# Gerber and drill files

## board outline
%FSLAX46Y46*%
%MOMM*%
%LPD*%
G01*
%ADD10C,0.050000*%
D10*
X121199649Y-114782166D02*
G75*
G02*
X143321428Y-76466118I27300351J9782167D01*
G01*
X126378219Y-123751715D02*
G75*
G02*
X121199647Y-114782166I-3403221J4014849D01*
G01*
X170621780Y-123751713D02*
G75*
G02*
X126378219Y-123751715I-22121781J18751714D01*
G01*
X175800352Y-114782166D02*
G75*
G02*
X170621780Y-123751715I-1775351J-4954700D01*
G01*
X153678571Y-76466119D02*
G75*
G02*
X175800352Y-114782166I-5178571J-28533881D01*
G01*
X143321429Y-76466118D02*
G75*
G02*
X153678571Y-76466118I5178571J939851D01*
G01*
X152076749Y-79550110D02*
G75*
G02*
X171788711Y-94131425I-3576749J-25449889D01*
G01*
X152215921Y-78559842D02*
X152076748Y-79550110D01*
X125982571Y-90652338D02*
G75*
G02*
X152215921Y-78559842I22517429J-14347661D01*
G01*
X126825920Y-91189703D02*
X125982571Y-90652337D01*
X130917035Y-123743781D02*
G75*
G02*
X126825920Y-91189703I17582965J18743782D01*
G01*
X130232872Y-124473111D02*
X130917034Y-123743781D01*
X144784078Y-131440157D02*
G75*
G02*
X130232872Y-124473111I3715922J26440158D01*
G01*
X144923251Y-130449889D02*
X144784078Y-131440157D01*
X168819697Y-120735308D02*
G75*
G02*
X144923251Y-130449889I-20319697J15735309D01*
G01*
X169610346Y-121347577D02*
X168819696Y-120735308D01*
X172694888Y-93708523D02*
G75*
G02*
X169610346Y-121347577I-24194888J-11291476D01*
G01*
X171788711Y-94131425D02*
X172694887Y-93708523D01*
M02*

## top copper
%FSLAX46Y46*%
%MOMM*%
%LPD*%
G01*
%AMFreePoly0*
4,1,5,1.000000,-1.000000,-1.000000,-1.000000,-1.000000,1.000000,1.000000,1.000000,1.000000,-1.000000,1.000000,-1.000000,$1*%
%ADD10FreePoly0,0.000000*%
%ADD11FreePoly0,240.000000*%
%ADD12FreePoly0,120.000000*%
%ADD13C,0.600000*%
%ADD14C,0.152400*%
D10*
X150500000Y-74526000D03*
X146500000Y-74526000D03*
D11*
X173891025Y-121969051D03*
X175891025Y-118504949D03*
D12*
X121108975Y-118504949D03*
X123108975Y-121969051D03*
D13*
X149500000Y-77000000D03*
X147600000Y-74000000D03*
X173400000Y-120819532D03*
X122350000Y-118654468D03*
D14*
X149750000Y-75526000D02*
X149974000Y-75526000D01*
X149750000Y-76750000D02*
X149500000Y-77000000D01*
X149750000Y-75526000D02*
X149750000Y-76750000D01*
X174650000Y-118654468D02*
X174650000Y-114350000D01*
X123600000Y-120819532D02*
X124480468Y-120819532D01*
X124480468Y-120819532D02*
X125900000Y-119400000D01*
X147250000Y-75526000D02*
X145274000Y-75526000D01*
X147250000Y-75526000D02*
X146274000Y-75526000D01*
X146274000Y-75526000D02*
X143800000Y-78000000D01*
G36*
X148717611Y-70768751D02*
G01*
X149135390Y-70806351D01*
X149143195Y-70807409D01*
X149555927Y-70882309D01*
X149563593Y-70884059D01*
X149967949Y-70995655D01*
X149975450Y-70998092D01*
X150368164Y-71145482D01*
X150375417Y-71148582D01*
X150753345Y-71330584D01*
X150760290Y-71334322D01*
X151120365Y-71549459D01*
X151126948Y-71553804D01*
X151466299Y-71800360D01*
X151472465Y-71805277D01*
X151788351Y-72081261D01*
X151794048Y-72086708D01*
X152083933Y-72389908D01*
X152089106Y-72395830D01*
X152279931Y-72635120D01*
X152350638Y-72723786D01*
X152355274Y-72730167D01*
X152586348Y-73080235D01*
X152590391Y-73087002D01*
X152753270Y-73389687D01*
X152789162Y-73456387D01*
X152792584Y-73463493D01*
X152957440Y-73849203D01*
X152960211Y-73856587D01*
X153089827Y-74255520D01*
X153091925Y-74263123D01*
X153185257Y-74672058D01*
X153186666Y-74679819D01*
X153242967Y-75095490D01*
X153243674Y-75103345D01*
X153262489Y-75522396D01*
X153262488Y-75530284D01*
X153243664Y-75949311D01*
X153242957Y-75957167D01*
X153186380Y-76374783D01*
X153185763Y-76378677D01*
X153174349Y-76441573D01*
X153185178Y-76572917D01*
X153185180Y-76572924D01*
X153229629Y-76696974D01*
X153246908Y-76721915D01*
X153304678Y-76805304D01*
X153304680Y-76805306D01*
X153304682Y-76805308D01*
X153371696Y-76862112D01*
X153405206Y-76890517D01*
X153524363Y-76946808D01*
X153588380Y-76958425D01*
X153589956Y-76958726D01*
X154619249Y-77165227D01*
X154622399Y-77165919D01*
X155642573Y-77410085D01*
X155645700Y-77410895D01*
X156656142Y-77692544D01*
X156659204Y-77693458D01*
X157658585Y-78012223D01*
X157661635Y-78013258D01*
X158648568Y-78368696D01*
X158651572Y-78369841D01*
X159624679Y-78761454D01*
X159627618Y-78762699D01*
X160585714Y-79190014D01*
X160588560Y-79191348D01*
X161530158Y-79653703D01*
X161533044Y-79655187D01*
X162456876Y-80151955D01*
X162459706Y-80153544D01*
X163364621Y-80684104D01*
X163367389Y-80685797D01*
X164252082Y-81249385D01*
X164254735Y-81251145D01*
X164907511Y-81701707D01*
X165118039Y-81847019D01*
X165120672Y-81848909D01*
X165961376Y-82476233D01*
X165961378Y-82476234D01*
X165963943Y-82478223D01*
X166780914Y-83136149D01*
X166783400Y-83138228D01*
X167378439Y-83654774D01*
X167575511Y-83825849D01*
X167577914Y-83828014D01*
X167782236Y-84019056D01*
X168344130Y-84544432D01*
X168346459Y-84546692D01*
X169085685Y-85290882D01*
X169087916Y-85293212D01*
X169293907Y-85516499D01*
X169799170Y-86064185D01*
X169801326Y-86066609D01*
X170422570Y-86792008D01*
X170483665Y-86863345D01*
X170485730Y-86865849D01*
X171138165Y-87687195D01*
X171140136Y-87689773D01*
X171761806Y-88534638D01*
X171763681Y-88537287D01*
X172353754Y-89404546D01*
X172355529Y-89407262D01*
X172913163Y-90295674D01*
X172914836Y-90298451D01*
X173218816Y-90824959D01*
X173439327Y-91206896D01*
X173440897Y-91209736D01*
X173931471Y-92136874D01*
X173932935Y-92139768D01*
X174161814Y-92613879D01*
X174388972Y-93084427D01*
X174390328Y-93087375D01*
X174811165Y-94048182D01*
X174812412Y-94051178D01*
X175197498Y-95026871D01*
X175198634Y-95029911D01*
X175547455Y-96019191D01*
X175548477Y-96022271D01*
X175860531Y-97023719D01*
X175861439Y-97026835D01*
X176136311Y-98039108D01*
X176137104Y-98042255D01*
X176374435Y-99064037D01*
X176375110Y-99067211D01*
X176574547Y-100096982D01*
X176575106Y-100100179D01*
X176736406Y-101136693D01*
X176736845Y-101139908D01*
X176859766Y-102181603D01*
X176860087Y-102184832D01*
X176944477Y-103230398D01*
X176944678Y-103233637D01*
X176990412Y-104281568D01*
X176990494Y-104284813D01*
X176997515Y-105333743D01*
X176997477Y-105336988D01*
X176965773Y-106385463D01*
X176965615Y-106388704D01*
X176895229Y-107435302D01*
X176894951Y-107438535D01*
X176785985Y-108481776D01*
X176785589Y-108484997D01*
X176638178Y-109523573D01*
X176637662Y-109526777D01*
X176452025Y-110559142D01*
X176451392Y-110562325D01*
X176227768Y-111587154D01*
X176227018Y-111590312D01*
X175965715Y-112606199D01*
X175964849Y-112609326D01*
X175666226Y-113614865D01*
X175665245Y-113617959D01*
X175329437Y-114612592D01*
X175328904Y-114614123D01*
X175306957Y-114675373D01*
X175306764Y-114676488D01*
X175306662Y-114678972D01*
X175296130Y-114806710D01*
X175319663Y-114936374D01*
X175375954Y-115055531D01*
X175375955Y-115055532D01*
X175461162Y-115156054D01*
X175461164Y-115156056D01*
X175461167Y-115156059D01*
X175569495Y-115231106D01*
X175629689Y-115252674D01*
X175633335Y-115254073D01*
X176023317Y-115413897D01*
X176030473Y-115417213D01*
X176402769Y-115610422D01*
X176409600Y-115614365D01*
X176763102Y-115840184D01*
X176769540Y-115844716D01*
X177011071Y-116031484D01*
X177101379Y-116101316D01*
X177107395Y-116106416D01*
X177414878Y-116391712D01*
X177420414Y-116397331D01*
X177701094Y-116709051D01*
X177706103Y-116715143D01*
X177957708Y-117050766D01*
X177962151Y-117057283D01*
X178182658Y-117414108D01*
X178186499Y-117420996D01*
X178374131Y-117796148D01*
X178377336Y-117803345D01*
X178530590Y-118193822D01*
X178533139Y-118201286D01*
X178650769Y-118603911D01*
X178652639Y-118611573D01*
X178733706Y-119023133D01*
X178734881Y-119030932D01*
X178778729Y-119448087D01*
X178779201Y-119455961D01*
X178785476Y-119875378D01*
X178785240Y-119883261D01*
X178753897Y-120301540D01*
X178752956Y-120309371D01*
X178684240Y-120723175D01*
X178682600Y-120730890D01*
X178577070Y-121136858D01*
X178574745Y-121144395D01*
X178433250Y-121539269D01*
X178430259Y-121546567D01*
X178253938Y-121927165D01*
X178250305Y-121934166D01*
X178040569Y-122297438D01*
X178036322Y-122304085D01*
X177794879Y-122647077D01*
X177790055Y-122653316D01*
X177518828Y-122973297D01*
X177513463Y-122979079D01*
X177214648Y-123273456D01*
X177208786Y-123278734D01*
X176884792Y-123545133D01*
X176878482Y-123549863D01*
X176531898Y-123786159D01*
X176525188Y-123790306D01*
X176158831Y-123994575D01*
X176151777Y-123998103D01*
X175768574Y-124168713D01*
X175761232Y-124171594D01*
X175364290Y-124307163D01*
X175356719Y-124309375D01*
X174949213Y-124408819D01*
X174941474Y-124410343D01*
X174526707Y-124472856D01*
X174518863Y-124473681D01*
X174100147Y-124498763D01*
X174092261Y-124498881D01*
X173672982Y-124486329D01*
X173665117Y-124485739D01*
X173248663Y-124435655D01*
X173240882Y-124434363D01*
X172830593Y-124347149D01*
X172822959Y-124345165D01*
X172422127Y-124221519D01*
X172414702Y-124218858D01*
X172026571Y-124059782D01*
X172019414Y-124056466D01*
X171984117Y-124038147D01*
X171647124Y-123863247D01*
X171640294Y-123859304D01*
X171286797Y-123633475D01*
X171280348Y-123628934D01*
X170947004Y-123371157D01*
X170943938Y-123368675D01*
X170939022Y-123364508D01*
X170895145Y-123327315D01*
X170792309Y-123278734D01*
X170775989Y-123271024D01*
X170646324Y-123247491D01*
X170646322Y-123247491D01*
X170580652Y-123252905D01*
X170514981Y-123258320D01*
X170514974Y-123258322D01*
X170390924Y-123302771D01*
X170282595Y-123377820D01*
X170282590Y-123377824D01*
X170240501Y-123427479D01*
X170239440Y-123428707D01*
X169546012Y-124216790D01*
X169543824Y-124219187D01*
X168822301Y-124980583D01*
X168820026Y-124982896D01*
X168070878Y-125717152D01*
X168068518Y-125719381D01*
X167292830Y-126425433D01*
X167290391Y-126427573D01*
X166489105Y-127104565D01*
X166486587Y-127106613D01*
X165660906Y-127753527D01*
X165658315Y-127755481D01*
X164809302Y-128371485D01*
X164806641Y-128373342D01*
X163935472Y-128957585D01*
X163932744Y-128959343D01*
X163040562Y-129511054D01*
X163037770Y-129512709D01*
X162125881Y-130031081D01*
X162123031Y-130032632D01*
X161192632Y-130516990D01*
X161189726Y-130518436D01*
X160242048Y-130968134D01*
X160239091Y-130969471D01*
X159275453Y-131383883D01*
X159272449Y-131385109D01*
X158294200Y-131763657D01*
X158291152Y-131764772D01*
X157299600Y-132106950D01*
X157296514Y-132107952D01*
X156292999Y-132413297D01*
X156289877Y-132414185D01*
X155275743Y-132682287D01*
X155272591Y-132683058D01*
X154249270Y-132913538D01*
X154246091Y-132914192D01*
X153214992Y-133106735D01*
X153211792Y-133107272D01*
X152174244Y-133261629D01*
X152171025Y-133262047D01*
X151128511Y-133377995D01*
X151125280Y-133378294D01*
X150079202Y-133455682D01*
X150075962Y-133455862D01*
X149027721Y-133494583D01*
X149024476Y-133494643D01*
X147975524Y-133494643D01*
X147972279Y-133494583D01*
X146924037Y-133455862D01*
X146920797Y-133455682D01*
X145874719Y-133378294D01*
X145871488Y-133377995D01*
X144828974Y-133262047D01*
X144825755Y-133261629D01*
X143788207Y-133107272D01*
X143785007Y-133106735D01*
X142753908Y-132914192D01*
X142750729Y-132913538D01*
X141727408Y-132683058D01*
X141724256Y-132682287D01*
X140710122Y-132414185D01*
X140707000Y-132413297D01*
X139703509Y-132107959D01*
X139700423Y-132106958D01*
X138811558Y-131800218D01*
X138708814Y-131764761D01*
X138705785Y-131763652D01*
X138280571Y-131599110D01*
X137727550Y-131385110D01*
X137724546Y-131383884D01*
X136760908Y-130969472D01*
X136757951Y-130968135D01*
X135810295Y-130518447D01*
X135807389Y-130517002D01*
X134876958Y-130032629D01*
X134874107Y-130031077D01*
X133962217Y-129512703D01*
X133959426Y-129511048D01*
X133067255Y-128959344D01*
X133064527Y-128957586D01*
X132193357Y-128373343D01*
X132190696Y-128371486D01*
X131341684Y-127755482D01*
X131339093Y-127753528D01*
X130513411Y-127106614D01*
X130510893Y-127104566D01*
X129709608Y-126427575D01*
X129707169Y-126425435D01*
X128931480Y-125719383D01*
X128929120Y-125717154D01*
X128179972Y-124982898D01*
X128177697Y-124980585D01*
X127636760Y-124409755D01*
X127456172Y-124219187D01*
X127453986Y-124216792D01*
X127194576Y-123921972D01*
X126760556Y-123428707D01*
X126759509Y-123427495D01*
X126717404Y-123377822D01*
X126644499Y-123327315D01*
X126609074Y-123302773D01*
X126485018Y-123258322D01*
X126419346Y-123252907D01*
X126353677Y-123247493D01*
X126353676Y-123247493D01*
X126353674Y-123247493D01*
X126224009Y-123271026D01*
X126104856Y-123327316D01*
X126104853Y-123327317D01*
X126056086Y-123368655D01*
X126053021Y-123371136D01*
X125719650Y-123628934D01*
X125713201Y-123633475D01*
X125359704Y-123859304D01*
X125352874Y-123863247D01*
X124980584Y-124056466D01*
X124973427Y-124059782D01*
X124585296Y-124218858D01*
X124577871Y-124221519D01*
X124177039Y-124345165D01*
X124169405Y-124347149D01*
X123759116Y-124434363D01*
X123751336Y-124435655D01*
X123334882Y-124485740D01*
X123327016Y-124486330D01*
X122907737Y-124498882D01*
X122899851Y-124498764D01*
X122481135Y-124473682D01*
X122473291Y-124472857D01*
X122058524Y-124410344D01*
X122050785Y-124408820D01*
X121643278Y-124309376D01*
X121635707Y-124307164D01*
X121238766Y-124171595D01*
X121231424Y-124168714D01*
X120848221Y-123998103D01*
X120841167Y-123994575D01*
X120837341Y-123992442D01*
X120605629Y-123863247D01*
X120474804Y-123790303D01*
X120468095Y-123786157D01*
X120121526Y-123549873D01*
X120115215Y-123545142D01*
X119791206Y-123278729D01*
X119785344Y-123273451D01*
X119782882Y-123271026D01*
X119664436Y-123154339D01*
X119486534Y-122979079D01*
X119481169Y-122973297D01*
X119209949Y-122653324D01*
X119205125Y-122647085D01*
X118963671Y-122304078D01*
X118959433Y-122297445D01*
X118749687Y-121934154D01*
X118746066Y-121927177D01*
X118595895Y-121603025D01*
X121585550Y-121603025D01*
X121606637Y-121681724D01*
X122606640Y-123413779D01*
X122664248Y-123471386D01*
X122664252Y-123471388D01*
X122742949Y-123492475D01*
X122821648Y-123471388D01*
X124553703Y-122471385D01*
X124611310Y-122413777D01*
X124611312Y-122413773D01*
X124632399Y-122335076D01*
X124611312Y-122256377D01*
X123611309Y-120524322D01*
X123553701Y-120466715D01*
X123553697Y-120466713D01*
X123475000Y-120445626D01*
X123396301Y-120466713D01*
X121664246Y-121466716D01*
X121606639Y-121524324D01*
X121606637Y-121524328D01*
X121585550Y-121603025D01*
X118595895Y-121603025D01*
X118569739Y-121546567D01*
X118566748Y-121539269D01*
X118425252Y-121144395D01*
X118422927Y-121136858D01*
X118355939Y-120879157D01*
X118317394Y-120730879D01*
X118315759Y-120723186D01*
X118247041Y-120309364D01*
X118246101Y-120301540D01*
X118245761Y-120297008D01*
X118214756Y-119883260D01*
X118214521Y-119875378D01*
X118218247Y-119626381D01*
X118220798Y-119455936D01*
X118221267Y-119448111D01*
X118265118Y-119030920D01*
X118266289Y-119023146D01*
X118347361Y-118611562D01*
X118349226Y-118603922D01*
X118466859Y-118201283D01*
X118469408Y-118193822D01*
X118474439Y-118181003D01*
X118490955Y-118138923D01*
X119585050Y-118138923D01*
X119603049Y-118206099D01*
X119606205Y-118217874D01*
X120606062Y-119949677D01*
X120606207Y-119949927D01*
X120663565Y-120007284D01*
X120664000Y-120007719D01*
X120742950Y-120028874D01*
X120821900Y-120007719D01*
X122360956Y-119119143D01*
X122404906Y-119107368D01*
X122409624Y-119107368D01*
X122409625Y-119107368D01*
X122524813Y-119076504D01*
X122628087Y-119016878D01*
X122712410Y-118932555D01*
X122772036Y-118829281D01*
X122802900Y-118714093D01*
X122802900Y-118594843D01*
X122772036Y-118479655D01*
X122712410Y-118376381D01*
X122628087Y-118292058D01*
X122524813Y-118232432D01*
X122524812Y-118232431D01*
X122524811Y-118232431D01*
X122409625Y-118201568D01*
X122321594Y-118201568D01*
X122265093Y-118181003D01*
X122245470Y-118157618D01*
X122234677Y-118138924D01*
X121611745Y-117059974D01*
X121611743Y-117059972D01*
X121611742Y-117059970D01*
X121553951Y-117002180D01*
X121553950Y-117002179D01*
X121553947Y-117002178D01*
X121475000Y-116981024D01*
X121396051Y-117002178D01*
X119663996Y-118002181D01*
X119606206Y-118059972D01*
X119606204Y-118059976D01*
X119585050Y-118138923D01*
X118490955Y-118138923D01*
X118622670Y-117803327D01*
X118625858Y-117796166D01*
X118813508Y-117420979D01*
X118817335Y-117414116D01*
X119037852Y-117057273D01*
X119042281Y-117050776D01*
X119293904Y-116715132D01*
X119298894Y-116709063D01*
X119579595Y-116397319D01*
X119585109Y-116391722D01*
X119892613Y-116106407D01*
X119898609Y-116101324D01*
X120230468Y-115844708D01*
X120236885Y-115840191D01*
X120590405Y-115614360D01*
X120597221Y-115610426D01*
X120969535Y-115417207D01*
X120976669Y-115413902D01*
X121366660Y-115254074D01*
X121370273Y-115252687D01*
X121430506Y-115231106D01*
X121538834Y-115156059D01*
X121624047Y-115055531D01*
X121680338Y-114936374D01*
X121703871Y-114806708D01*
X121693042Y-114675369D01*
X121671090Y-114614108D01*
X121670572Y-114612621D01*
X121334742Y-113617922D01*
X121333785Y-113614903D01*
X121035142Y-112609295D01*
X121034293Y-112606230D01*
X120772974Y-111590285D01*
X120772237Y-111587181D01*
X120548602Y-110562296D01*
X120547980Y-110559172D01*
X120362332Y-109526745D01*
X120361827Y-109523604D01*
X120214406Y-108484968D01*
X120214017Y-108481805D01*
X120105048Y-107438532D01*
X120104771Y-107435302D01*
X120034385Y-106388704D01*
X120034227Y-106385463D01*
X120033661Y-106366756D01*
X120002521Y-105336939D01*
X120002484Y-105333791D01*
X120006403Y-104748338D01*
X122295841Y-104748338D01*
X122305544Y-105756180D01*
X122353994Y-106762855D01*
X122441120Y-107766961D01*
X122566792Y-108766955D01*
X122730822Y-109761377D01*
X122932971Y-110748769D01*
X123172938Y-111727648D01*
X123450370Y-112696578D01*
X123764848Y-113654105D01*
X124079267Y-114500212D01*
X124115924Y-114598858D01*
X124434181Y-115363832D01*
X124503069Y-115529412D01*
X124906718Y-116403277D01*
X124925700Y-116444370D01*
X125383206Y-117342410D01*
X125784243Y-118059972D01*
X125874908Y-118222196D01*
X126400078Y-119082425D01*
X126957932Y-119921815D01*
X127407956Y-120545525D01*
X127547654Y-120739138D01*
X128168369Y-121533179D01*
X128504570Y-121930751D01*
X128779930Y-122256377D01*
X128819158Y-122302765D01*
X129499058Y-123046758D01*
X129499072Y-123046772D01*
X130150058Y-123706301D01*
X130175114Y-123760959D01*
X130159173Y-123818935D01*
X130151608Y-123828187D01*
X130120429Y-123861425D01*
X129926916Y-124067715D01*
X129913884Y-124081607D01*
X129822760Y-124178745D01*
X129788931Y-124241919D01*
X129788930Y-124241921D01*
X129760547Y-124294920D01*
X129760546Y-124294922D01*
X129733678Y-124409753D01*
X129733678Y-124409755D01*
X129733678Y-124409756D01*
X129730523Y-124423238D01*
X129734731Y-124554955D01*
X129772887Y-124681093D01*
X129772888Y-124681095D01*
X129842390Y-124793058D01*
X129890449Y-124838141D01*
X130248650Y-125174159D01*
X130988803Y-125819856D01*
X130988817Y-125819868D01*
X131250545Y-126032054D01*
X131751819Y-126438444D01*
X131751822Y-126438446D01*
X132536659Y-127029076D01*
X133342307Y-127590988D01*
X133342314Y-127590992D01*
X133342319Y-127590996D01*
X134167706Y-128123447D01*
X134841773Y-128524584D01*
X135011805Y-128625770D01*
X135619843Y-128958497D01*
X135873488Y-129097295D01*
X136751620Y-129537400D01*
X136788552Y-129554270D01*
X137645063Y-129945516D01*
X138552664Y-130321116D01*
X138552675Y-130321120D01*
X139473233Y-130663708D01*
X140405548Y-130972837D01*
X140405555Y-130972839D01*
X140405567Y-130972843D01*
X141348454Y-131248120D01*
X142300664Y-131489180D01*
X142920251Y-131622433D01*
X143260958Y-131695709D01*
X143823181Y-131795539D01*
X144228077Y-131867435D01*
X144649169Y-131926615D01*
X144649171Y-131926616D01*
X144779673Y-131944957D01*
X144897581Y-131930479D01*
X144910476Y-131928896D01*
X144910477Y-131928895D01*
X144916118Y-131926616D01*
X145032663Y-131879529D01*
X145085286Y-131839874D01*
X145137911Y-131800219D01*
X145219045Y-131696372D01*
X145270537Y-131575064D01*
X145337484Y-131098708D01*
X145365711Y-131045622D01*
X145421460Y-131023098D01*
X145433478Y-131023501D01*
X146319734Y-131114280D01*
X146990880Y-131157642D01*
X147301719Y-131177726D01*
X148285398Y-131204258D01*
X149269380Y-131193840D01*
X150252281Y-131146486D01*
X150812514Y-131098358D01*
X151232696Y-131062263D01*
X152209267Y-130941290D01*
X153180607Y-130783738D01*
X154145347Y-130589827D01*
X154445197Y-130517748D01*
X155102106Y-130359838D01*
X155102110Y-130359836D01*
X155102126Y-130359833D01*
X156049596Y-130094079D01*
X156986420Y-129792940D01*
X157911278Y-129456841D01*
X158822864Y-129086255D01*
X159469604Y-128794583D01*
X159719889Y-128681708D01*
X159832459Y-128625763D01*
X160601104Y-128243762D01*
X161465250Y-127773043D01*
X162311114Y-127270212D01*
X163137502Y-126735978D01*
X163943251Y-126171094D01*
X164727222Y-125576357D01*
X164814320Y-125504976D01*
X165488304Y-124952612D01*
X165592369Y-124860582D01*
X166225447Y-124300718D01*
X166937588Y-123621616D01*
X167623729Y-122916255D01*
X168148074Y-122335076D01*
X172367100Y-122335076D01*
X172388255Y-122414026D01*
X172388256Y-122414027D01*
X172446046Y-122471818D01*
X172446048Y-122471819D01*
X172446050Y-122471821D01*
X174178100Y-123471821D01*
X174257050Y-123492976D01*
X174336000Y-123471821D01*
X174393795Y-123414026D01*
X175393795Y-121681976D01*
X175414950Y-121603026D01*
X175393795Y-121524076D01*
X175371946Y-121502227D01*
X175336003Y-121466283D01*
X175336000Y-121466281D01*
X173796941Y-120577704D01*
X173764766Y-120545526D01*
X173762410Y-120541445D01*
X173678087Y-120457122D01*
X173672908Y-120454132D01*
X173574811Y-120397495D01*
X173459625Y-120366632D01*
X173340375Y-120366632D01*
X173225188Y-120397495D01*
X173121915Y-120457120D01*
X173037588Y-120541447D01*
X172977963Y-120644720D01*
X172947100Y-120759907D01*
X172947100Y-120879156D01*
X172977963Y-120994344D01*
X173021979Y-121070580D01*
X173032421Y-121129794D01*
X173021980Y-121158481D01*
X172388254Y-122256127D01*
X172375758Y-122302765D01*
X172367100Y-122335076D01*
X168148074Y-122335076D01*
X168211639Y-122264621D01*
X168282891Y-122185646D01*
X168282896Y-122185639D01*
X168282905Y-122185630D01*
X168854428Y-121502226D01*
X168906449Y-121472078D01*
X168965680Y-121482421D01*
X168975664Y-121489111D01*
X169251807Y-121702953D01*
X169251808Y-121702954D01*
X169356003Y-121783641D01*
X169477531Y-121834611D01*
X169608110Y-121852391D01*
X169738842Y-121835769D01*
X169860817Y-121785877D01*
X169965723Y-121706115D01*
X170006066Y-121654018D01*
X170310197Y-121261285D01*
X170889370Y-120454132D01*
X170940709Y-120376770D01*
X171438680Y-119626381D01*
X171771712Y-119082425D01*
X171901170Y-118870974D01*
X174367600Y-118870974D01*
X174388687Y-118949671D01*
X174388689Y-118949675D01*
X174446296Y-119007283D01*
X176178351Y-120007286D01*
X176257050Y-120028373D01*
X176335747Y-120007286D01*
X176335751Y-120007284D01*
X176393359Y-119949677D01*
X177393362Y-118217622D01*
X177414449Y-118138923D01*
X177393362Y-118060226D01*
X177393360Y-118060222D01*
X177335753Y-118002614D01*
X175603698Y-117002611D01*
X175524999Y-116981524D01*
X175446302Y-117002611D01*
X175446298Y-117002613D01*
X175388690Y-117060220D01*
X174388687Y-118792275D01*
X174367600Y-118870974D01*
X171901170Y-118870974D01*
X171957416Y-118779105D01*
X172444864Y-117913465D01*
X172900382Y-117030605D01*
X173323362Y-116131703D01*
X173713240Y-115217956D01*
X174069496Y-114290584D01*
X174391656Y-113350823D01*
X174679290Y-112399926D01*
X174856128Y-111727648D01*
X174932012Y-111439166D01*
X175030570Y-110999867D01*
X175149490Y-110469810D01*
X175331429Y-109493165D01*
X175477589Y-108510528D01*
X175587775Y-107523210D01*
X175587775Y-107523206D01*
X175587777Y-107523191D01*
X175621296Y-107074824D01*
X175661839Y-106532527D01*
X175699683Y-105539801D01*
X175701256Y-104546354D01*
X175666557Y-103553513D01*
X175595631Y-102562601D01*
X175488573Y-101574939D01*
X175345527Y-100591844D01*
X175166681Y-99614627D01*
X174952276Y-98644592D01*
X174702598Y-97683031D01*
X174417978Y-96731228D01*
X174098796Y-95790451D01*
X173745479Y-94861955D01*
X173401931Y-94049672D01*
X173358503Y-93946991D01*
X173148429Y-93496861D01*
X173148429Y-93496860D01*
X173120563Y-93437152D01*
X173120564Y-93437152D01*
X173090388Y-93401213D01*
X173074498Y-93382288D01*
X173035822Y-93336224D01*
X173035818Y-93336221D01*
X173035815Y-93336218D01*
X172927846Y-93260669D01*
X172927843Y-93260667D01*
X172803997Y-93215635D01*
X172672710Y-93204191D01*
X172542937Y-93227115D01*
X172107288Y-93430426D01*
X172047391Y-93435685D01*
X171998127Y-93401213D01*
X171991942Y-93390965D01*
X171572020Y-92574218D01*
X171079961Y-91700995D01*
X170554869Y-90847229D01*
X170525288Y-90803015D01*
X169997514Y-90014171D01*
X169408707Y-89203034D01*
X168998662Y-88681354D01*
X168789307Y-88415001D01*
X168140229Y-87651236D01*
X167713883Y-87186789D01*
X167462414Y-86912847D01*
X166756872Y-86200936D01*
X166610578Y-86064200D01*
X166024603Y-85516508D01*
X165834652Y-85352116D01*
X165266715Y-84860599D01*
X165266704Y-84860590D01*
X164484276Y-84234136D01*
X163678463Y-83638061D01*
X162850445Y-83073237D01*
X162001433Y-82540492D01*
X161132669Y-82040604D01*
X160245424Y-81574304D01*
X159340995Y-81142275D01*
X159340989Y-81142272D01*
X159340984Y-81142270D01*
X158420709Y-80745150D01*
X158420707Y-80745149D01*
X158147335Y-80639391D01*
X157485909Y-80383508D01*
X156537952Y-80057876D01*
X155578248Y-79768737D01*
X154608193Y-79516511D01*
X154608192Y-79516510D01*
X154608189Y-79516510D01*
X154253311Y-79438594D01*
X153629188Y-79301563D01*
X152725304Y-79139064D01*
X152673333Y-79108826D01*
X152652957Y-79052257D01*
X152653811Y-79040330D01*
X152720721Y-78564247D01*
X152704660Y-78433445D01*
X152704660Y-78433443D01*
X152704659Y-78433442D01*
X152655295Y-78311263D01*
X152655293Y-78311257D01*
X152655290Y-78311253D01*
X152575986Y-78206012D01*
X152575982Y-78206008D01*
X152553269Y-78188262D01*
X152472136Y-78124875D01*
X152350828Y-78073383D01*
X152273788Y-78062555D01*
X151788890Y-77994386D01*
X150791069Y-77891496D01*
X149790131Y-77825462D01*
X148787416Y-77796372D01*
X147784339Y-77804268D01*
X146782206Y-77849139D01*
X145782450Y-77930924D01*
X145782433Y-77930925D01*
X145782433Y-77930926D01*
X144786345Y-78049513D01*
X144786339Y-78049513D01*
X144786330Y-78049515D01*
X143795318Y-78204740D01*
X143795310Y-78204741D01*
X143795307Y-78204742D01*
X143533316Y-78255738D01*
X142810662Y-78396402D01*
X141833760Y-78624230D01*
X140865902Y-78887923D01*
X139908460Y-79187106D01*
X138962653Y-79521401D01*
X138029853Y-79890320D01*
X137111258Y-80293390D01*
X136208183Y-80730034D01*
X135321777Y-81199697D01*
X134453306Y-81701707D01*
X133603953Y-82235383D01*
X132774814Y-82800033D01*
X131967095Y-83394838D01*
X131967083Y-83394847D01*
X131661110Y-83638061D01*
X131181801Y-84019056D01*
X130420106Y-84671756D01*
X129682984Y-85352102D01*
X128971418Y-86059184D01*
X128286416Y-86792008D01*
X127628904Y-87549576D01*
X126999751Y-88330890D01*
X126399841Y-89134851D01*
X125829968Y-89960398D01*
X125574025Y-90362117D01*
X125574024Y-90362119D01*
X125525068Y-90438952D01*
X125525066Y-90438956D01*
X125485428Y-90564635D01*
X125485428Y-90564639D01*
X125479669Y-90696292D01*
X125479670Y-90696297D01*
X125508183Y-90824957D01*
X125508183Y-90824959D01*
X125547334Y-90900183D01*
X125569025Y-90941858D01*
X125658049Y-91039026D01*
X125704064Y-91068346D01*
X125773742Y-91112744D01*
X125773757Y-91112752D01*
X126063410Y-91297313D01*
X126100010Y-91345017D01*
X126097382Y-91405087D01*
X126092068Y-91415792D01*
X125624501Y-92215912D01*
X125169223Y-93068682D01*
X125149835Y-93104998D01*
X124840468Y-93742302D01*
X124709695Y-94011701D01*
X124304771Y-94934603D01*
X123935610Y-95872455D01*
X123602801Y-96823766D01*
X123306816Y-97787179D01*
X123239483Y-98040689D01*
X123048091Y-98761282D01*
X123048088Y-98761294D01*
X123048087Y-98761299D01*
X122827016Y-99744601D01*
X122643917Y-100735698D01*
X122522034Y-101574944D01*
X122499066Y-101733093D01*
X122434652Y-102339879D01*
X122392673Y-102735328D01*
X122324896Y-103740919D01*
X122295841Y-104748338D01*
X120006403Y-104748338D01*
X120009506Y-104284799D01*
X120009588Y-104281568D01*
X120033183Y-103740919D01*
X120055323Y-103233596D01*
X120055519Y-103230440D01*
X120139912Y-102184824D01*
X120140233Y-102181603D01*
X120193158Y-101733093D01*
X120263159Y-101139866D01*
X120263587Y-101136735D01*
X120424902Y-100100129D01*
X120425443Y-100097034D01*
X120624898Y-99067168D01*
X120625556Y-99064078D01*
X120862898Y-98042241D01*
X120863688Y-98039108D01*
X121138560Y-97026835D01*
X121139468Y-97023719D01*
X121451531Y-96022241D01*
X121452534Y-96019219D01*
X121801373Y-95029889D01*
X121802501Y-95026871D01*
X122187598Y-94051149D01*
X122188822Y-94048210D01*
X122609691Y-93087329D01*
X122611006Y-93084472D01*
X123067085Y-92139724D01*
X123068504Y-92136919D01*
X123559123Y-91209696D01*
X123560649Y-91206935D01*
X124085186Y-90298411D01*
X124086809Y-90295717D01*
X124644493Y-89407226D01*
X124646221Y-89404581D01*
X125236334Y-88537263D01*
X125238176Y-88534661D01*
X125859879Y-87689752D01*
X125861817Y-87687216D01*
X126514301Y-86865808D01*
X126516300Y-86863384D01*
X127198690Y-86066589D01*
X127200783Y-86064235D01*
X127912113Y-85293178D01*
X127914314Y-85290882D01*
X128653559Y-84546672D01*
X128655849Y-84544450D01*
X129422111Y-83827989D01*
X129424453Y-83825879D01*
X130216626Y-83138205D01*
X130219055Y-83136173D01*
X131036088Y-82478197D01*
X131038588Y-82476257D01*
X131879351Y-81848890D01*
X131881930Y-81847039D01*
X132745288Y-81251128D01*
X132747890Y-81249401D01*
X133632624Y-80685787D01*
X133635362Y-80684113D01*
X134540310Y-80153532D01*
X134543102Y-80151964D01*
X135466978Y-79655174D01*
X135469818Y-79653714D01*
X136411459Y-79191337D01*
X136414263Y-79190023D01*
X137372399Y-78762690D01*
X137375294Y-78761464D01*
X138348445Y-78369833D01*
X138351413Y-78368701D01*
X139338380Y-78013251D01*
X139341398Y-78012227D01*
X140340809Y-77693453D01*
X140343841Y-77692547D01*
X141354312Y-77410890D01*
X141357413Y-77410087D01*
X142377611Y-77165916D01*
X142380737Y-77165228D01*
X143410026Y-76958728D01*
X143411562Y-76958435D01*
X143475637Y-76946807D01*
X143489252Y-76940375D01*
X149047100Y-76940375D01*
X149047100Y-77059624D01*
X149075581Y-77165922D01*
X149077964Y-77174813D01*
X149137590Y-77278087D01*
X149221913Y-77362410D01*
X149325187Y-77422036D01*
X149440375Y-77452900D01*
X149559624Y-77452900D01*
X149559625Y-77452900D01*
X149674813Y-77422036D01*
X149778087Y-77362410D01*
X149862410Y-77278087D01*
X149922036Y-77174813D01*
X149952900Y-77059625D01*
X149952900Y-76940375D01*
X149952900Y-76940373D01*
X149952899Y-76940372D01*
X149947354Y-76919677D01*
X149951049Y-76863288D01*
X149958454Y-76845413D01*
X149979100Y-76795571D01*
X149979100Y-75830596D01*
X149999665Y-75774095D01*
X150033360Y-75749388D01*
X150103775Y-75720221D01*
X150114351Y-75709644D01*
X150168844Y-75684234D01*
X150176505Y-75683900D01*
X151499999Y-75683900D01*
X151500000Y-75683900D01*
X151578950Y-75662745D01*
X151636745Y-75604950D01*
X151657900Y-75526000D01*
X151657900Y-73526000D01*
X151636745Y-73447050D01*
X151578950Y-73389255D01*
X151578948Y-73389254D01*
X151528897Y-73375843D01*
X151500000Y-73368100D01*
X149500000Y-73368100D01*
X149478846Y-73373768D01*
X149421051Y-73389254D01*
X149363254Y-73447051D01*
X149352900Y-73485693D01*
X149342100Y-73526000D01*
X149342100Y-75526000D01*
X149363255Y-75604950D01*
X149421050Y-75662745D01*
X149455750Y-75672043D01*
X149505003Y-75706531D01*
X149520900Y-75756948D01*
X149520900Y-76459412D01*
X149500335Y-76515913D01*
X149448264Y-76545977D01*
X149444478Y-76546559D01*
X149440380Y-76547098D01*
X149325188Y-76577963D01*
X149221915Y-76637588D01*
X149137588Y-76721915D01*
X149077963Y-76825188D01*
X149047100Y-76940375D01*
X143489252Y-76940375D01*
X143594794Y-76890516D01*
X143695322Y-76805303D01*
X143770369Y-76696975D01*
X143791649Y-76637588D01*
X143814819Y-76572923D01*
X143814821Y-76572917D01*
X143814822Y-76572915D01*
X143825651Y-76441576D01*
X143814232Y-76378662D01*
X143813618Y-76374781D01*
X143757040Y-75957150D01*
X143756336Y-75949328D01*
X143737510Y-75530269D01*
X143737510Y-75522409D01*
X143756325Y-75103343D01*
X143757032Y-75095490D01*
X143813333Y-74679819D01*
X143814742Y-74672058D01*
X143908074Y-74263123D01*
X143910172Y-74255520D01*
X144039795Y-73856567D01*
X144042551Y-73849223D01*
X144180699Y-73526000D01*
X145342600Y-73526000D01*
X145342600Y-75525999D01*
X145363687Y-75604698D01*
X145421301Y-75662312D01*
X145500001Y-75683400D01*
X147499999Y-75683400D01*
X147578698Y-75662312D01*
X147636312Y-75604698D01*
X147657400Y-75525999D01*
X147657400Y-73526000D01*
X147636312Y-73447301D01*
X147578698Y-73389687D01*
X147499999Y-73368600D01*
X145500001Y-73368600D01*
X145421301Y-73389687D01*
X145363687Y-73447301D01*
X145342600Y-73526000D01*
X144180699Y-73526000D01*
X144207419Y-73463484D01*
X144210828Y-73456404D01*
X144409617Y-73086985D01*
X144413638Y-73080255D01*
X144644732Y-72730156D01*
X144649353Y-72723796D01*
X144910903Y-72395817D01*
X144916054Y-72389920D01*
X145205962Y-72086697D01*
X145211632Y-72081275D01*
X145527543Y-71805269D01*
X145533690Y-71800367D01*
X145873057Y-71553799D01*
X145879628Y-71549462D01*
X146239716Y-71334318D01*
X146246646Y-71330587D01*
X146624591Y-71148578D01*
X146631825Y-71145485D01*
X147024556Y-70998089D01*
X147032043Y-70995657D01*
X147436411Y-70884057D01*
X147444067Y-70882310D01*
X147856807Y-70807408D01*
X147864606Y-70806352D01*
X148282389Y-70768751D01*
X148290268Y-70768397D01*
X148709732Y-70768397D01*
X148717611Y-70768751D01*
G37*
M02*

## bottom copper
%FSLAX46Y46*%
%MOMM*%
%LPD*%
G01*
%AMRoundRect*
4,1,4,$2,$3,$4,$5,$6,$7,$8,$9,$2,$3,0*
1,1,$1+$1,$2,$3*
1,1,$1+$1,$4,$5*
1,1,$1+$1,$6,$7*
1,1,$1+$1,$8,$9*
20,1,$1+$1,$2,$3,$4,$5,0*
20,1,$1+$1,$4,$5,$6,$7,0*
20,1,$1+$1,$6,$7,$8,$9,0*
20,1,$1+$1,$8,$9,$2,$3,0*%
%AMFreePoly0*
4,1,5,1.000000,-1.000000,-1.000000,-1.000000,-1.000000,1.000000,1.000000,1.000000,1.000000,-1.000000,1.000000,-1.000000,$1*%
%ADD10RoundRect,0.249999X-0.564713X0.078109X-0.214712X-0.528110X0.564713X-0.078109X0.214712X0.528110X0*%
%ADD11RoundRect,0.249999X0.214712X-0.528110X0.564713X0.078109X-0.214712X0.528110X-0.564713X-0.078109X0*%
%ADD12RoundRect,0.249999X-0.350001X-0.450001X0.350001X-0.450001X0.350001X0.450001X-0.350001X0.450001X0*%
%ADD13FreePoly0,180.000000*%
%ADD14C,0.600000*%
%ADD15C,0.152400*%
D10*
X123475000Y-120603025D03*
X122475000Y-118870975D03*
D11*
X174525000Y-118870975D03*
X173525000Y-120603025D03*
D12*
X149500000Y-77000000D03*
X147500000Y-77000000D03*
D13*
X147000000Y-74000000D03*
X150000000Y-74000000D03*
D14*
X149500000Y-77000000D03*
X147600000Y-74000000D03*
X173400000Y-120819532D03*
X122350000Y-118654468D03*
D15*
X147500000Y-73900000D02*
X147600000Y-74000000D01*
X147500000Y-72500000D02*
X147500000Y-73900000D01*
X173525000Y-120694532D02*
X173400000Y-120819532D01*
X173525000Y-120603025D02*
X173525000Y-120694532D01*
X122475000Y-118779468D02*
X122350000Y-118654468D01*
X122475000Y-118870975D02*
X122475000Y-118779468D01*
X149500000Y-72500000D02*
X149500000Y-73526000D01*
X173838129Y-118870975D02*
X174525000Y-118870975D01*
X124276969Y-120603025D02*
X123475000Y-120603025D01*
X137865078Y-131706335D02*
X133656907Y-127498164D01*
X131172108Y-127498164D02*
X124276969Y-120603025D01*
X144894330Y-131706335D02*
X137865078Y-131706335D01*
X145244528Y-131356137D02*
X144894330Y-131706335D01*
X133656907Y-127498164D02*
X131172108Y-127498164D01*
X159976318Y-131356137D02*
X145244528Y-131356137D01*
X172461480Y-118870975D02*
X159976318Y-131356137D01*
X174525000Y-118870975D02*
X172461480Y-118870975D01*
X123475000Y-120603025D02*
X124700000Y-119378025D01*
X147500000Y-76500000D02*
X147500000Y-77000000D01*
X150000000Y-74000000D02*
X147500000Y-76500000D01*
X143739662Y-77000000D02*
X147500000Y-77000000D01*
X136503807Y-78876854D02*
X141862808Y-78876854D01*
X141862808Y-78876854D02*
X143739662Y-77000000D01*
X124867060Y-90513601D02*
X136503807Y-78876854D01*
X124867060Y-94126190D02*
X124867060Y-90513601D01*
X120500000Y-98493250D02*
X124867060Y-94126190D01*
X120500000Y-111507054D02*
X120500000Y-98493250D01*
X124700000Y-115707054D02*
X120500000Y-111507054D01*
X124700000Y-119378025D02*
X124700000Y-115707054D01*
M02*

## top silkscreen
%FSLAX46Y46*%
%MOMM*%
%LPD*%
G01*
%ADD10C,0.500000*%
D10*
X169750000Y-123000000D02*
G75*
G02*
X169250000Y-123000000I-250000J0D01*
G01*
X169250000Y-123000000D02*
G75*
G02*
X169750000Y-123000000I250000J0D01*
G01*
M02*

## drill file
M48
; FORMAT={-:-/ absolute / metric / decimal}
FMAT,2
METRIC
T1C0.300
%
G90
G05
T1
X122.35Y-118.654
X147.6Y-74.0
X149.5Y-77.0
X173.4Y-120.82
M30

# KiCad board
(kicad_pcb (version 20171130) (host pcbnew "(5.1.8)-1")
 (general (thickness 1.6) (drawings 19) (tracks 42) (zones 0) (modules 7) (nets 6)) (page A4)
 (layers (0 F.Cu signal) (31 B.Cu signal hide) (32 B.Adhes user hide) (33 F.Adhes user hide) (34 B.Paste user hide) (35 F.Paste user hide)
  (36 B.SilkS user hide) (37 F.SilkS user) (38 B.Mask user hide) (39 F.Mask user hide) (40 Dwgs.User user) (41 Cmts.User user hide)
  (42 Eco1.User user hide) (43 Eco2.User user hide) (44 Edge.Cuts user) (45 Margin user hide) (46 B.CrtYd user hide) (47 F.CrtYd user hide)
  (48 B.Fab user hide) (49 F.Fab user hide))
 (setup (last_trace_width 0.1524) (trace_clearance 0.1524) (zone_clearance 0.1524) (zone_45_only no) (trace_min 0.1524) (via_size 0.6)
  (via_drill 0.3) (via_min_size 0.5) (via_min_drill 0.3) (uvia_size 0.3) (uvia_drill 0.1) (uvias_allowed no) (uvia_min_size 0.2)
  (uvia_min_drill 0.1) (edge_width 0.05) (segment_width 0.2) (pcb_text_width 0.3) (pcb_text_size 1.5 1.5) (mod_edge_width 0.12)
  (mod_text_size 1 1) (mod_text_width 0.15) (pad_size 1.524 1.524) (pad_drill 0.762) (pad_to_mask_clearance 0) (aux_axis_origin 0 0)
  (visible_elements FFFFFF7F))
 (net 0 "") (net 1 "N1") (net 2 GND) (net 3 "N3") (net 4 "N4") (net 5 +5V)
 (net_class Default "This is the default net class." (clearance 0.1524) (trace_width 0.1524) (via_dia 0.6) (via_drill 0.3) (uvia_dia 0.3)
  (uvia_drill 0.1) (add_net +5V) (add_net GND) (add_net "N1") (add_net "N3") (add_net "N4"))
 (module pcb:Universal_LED (layer F.Cu) (at 148.5 75.526)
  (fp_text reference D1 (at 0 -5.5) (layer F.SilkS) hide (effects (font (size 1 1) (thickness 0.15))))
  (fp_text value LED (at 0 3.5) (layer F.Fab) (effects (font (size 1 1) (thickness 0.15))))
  (pad 2 smd custom (at 2 -1) (size 2 2) (layers F.Cu F.Paste F.Mask) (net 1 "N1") (zone_connect 0)
   (options (clearance outline) (anchor rect)) (primitives))
  (pad 1 smd custom (at -2 -1) (size 2 2) (layers F.Cu F.Paste F.Mask) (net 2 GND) (zone_connect 0)
   (options (clearance outline) (anchor rect)) (primitives)))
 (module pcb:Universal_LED (layer F.Cu) (at 174.025 119.737 240)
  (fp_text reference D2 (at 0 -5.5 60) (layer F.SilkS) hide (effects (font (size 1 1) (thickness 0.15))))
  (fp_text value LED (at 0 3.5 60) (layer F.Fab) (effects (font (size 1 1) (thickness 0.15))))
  (pad 2 smd custom (at 2 -1 240) (size 2 2) (layers F.Cu F.Paste F.Mask) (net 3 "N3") (zone_connect 0)
   (options (clearance outline) (anchor rect)) (primitives))
  (pad 1 smd custom (at -2 -1 240) (size 2 2) (layers F.Cu F.Paste F.Mask) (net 2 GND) (zone_connect 0)
   (options (clearance outline) (anchor rect)) (primitives)))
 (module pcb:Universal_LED (layer F.Cu) (at 122.975 119.737 120)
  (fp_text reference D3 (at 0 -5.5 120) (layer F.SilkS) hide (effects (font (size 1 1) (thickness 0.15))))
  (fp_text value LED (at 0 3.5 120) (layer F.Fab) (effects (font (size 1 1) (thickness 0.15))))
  (pad 2 smd custom (at 2 -1 120) (size 2 2) (layers F.Cu F.Paste F.Mask) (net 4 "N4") (zone_connect 0)
   (options (clearance outline) (anchor rect)) (primitives))
  (pad 1 smd custom (at -2 -1 120) (size 2 2) (layers F.Cu F.Paste F.Mask) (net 2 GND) (zone_connect 0)
   (options (clearance outline) (anchor rect)) (primitives)))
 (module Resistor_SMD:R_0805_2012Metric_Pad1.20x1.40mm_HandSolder (layer B.Cu) (at 122.975 119.737 300)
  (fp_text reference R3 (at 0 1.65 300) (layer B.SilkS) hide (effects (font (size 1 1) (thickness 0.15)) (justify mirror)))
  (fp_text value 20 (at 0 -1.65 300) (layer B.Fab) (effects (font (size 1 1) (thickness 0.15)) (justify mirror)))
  (pad 2 smd roundrect (at 1 0 300) (size 1.2 1.4) (layers B.Cu B.Paste B.Mask) (roundrect_rratio 0.2083325) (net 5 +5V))
  (pad 1 smd roundrect (at -1 0 300) (size 1.2 1.4) (layers B.Cu B.Paste B.Mask) (roundrect_rratio 0.2083325) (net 4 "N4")))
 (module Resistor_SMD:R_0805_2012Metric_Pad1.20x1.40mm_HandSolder (layer B.Cu) (at 174.025 119.737 60)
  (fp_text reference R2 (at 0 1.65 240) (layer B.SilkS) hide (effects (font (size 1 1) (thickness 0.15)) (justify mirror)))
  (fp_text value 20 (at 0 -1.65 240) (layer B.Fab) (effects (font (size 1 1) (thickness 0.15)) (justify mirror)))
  (pad 2 smd roundrect (at 1 0 60) (size 1.2 1.4) (layers B.Cu B.Paste B.Mask) (roundrect_rratio 0.2083325) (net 5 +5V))
  (pad 1 smd roundrect (at -1 0 60) (size 1.2 1.4) (layers B.Cu B.Paste B.Mask) (roundrect_rratio 0.2083325) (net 3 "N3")))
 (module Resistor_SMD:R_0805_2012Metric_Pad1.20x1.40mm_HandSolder (layer B.Cu) (at 148.5 77)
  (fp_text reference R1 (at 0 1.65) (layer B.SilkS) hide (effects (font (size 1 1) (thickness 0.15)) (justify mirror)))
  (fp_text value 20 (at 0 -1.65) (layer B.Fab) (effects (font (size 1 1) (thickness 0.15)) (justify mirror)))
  (pad 2 smd roundrect (at 1 0) (size 1.2 1.4) (layers B.Cu B.Paste B.Mask) (roundrect_rratio 0.2083325) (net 1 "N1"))
  (pad 1 smd roundrect (at -1 0) (size 1.2 1.4) (layers B.Cu B.Paste B.Mask) (roundrect_rratio 0.2083325) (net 5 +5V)))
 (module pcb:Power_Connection (layer B.Cu) (at 148.5 75.5 180)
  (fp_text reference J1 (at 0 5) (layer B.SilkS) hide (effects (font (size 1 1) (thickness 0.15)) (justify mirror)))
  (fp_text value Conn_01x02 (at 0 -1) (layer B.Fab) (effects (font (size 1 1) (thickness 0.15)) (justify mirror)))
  (pad 1 smd custom (at 1.5 1.5 180) (size 2 2) (layers B.Cu B.Paste B.Mask) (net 2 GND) (zone_connect 0)
   (options (clearance outline) (anchor rect)) (primitives))
  (pad 2 smd custom (at -1.5 1.5 180) (size 2 2) (layers B.Cu B.Paste B.Mask) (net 5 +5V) (zone_connect 0)
   (options (clearance outline) (anchor rect)) (primitives)))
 (gr_circle (center 169.5 123) (end 169.75 123) (layer F.SilkS) (width 0.5))
 (gr_arc (start 148.5 104.999999) (end 143.321428 76.466118) (angle -99.42687878) (layer Edge.Cuts) (width 0.05))
 (gr_arc (start 122.974998 119.736866) (end 121.199647 114.782166) (angle -200.5731212) (layer Edge.Cuts) (width 0.05))
 (gr_arc (start 148.499999 104.999999) (end 126.378219 123.751715) (angle -99.42687878) (layer Edge.Cuts) (width 0.05))
 (gr_arc (start 174.025001 119.736866) (end 170.62178 123.751715) (angle -200.5731212) (layer Edge.Cuts) (width 0.05))
 (gr_arc (start 148.5 105) (end 175.800352 114.782166) (angle -99.42687878) (layer Edge.Cuts) (width 0.05))
 (gr_arc (start 148.5 75.526267) (end 153.678571 76.466118) (angle -200.5731212) (layer Edge.Cuts) (width 0.05))
 (gr_arc (start 148.5 104.999999) (end 171.788711 94.131425) (angle -56.98207807) (layer Edge.Cuts) (width 0.05))
 (gr_line (start 152.215921 78.559842) (end 152.076748 79.55011) (layer Edge.Cuts) (width 0.05))
 (gr_arc (start 148.5 104.999999) (end 152.215921 78.559842) (angle -65.49551528) (layer Edge.Cuts) (width 0.05))
 (gr_line (start 126.82592 91.189703) (end 125.982571 90.652337) (layer Edge.Cuts) (width 0.05))
 (gr_arc (start 148.5 104.999999) (end 126.82592 91.189703) (angle -79.33474074) (layer Edge.Cuts) (width 0.05))
 (gr_line (start 130.232872 124.473111) (end 130.917034 123.743781) (layer Edge.Cuts) (width 0.05))
 (gr_arc (start 148.5 104.999999) (end 130.232872 124.473111) (angle -35.16974396) (layer Edge.Cuts) (width 0.05))
 (gr_line (start 144.923251 130.449889) (end 144.784078 131.440157) (layer Edge.Cuts) (width 0.05))
 (gr_arc (start 148.5 104.999999) (end 144.923251 130.449889) (angle -60.24626543) (layer Edge.Cuts) (width 0.05))
 (gr_line (start 169.610346 121.347577) (end 168.819696 120.735308) (layer Edge.Cuts) (width 0.05))
 (gr_arc (start 148.5 104.999999) (end 169.610346 121.347577) (angle -62.77165651) (layer Edge.Cuts) (width 0.05))
 (gr_line (start 171.788711 94.131425) (end 172.694887 93.708523) (layer Edge.Cuts) (width 0.05))
 (segment (start 149.75 75.526) (end 149.974 75.526) (width 0.1524) (layer F.Cu) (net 1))
 (via (at 149.5 77) (size 0.6) (drill 0.3) (layers F.Cu B.Cu) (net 1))
 (segment (start 149.75 76.75) (end 149.5 77) (width 0.1524) (layer F.Cu) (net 1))
 (segment (start 149.75 75.526) (end 149.75 76.75) (width 0.1524) (layer F.Cu) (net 1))
 (segment (start 174.65 118.654468) (end 174.65 114.35) (width 0.1524) (layer F.Cu) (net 2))
 (segment (start 123.6 120.819532) (end 124.480468 120.819532) (width 0.1524) (layer F.Cu) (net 2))
 (segment (start 124.480468 120.819532) (end 125.9 119.4) (width 0.1524) (layer F.Cu) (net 2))
 (segment (start 147.25 75.526) (end 145.274 75.526) (width 0.1524) (layer F.Cu) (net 2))
 (segment (start 147.25 75.526) (end 146.274 75.526) (width 0.1524) (layer F.Cu) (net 2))
 (segment (start 147.5 73.9) (end 147.6 74) (width 0.1524) (layer B.Cu) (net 2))
 (segment (start 147.5 72.5) (end 147.5 73.9) (width 0.1524) (layer B.Cu) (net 2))
 (via (at 147.6 74) (size 0.6) (drill 0.3) (layers F.Cu B.Cu) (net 2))
 (segment (start 146.274 75.526) (end 143.8 78) (width 0.1524) (layer F.Cu) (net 2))
 (via (at 173.4 120.819532) (size 0.6) (drill 0.3) (layers F.Cu B.Cu) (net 3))
 (segment (start 173.525 120.694532) (end 173.4 120.819532) (width 0.1524) (layer B.Cu) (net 3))
 (segment (start 173.525 120.603025) (end 173.525 120.694532) (width 0.1524) (layer B.Cu) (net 3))
 (via (at 122.35 118.654468) (size 0.6) (drill 0.3) (layers F.Cu B.Cu) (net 4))
 (segment (start 122.475 118.779468) (end 122.35 118.654468) (width 0.1524) (layer B.Cu) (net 4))
 (segment (start 122.475 118.870975) (end 122.475 118.779468) (width 0.1524) (layer B.Cu) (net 4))
 (segment (start 149.5 72.5) (end 149.5 73.526) (width 0.1524) (layer B.Cu) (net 5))
 (segment (start 173.838129 118.870975) (end 174.525 118.870975) (width 0.1524) (layer B.Cu) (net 5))
 (segment (start 124.276969 120.603025) (end 123.475 120.603025) (width 0.1524) (layer B.Cu) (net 5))
 (segment (start 137.865078 131.706335) (end 133.656907 127.498164) (width 0.1524) (layer B.Cu) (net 5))
 (segment (start 131.172108 127.498164) (end 124.276969 120.603025) (width 0.1524) (layer B.Cu) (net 5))
 (segment (start 144.89433 131.706335) (end 137.865078 131.706335) (width 0.1524) (layer B.Cu) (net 5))
 (segment (start 145.244528 131.356137) (end 144.89433 131.706335) (width 0.1524) (layer B.Cu) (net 5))
 (segment (start 133.656907 127.498164) (end 131.172108 127.498164) (width 0.1524) (layer B.Cu) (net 5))
 (segment (start 159.976318 131.356137) (end 145.244528 131.356137) (width 0.1524) (layer B.Cu) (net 5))
 (segment (start 172.46148 118.870975) (end 159.976318 131.356137) (width 0.1524) (layer B.Cu) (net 5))
 (segment (start 174.525 118.870975) (end 172.46148 118.870975) (width 0.1524) (layer B.Cu) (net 5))
 (segment (start 123.475 120.603025) (end 124.7 119.378025) (width 0.1524) (layer B.Cu) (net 5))
 (segment (start 147.5 76.5) (end 147.5 77) (width 0.1524) (layer B.Cu) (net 5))
 (segment (start 150 74) (end 147.5 76.5) (width 0.1524) (layer B.Cu) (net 5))
 (segment (start 143.739662 77) (end 147.5 77) (width 0.1524) (layer B.Cu) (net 5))
 (segment (start 136.503807 78.876854) (end 141.862808 78.876854) (width 0.1524) (layer B.Cu) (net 5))
 (segment (start 141.862808 78.876854) (end 143.739662 77) (width 0.1524) (layer B.Cu) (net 5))
 (segment (start 124.86706 90.513601) (end 136.503807 78.876854) (width 0.1524) (layer B.Cu) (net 5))
 (segment (start 124.86706 94.12619) (end 124.86706 90.513601) (width 0.1524) (layer B.Cu) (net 5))
 (segment (start 120.5 98.49325) (end 124.86706 94.12619) (width 0.1524) (layer B.Cu) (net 5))
 (segment (start 120.5 111.507054) (end 120.5 98.49325) (width 0.1524) (layer B.Cu) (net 5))
 (segment (start 124.7 115.707054) (end 120.5 111.507054) (width 0.1524) (layer B.Cu) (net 5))
 (segment (start 124.7 119.378025) (end 124.7 115.707054) (width 0.1524) (layer B.Cu) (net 5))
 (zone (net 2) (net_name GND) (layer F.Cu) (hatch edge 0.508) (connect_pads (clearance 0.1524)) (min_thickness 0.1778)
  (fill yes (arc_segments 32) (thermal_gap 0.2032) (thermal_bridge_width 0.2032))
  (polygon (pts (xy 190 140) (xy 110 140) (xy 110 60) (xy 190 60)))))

